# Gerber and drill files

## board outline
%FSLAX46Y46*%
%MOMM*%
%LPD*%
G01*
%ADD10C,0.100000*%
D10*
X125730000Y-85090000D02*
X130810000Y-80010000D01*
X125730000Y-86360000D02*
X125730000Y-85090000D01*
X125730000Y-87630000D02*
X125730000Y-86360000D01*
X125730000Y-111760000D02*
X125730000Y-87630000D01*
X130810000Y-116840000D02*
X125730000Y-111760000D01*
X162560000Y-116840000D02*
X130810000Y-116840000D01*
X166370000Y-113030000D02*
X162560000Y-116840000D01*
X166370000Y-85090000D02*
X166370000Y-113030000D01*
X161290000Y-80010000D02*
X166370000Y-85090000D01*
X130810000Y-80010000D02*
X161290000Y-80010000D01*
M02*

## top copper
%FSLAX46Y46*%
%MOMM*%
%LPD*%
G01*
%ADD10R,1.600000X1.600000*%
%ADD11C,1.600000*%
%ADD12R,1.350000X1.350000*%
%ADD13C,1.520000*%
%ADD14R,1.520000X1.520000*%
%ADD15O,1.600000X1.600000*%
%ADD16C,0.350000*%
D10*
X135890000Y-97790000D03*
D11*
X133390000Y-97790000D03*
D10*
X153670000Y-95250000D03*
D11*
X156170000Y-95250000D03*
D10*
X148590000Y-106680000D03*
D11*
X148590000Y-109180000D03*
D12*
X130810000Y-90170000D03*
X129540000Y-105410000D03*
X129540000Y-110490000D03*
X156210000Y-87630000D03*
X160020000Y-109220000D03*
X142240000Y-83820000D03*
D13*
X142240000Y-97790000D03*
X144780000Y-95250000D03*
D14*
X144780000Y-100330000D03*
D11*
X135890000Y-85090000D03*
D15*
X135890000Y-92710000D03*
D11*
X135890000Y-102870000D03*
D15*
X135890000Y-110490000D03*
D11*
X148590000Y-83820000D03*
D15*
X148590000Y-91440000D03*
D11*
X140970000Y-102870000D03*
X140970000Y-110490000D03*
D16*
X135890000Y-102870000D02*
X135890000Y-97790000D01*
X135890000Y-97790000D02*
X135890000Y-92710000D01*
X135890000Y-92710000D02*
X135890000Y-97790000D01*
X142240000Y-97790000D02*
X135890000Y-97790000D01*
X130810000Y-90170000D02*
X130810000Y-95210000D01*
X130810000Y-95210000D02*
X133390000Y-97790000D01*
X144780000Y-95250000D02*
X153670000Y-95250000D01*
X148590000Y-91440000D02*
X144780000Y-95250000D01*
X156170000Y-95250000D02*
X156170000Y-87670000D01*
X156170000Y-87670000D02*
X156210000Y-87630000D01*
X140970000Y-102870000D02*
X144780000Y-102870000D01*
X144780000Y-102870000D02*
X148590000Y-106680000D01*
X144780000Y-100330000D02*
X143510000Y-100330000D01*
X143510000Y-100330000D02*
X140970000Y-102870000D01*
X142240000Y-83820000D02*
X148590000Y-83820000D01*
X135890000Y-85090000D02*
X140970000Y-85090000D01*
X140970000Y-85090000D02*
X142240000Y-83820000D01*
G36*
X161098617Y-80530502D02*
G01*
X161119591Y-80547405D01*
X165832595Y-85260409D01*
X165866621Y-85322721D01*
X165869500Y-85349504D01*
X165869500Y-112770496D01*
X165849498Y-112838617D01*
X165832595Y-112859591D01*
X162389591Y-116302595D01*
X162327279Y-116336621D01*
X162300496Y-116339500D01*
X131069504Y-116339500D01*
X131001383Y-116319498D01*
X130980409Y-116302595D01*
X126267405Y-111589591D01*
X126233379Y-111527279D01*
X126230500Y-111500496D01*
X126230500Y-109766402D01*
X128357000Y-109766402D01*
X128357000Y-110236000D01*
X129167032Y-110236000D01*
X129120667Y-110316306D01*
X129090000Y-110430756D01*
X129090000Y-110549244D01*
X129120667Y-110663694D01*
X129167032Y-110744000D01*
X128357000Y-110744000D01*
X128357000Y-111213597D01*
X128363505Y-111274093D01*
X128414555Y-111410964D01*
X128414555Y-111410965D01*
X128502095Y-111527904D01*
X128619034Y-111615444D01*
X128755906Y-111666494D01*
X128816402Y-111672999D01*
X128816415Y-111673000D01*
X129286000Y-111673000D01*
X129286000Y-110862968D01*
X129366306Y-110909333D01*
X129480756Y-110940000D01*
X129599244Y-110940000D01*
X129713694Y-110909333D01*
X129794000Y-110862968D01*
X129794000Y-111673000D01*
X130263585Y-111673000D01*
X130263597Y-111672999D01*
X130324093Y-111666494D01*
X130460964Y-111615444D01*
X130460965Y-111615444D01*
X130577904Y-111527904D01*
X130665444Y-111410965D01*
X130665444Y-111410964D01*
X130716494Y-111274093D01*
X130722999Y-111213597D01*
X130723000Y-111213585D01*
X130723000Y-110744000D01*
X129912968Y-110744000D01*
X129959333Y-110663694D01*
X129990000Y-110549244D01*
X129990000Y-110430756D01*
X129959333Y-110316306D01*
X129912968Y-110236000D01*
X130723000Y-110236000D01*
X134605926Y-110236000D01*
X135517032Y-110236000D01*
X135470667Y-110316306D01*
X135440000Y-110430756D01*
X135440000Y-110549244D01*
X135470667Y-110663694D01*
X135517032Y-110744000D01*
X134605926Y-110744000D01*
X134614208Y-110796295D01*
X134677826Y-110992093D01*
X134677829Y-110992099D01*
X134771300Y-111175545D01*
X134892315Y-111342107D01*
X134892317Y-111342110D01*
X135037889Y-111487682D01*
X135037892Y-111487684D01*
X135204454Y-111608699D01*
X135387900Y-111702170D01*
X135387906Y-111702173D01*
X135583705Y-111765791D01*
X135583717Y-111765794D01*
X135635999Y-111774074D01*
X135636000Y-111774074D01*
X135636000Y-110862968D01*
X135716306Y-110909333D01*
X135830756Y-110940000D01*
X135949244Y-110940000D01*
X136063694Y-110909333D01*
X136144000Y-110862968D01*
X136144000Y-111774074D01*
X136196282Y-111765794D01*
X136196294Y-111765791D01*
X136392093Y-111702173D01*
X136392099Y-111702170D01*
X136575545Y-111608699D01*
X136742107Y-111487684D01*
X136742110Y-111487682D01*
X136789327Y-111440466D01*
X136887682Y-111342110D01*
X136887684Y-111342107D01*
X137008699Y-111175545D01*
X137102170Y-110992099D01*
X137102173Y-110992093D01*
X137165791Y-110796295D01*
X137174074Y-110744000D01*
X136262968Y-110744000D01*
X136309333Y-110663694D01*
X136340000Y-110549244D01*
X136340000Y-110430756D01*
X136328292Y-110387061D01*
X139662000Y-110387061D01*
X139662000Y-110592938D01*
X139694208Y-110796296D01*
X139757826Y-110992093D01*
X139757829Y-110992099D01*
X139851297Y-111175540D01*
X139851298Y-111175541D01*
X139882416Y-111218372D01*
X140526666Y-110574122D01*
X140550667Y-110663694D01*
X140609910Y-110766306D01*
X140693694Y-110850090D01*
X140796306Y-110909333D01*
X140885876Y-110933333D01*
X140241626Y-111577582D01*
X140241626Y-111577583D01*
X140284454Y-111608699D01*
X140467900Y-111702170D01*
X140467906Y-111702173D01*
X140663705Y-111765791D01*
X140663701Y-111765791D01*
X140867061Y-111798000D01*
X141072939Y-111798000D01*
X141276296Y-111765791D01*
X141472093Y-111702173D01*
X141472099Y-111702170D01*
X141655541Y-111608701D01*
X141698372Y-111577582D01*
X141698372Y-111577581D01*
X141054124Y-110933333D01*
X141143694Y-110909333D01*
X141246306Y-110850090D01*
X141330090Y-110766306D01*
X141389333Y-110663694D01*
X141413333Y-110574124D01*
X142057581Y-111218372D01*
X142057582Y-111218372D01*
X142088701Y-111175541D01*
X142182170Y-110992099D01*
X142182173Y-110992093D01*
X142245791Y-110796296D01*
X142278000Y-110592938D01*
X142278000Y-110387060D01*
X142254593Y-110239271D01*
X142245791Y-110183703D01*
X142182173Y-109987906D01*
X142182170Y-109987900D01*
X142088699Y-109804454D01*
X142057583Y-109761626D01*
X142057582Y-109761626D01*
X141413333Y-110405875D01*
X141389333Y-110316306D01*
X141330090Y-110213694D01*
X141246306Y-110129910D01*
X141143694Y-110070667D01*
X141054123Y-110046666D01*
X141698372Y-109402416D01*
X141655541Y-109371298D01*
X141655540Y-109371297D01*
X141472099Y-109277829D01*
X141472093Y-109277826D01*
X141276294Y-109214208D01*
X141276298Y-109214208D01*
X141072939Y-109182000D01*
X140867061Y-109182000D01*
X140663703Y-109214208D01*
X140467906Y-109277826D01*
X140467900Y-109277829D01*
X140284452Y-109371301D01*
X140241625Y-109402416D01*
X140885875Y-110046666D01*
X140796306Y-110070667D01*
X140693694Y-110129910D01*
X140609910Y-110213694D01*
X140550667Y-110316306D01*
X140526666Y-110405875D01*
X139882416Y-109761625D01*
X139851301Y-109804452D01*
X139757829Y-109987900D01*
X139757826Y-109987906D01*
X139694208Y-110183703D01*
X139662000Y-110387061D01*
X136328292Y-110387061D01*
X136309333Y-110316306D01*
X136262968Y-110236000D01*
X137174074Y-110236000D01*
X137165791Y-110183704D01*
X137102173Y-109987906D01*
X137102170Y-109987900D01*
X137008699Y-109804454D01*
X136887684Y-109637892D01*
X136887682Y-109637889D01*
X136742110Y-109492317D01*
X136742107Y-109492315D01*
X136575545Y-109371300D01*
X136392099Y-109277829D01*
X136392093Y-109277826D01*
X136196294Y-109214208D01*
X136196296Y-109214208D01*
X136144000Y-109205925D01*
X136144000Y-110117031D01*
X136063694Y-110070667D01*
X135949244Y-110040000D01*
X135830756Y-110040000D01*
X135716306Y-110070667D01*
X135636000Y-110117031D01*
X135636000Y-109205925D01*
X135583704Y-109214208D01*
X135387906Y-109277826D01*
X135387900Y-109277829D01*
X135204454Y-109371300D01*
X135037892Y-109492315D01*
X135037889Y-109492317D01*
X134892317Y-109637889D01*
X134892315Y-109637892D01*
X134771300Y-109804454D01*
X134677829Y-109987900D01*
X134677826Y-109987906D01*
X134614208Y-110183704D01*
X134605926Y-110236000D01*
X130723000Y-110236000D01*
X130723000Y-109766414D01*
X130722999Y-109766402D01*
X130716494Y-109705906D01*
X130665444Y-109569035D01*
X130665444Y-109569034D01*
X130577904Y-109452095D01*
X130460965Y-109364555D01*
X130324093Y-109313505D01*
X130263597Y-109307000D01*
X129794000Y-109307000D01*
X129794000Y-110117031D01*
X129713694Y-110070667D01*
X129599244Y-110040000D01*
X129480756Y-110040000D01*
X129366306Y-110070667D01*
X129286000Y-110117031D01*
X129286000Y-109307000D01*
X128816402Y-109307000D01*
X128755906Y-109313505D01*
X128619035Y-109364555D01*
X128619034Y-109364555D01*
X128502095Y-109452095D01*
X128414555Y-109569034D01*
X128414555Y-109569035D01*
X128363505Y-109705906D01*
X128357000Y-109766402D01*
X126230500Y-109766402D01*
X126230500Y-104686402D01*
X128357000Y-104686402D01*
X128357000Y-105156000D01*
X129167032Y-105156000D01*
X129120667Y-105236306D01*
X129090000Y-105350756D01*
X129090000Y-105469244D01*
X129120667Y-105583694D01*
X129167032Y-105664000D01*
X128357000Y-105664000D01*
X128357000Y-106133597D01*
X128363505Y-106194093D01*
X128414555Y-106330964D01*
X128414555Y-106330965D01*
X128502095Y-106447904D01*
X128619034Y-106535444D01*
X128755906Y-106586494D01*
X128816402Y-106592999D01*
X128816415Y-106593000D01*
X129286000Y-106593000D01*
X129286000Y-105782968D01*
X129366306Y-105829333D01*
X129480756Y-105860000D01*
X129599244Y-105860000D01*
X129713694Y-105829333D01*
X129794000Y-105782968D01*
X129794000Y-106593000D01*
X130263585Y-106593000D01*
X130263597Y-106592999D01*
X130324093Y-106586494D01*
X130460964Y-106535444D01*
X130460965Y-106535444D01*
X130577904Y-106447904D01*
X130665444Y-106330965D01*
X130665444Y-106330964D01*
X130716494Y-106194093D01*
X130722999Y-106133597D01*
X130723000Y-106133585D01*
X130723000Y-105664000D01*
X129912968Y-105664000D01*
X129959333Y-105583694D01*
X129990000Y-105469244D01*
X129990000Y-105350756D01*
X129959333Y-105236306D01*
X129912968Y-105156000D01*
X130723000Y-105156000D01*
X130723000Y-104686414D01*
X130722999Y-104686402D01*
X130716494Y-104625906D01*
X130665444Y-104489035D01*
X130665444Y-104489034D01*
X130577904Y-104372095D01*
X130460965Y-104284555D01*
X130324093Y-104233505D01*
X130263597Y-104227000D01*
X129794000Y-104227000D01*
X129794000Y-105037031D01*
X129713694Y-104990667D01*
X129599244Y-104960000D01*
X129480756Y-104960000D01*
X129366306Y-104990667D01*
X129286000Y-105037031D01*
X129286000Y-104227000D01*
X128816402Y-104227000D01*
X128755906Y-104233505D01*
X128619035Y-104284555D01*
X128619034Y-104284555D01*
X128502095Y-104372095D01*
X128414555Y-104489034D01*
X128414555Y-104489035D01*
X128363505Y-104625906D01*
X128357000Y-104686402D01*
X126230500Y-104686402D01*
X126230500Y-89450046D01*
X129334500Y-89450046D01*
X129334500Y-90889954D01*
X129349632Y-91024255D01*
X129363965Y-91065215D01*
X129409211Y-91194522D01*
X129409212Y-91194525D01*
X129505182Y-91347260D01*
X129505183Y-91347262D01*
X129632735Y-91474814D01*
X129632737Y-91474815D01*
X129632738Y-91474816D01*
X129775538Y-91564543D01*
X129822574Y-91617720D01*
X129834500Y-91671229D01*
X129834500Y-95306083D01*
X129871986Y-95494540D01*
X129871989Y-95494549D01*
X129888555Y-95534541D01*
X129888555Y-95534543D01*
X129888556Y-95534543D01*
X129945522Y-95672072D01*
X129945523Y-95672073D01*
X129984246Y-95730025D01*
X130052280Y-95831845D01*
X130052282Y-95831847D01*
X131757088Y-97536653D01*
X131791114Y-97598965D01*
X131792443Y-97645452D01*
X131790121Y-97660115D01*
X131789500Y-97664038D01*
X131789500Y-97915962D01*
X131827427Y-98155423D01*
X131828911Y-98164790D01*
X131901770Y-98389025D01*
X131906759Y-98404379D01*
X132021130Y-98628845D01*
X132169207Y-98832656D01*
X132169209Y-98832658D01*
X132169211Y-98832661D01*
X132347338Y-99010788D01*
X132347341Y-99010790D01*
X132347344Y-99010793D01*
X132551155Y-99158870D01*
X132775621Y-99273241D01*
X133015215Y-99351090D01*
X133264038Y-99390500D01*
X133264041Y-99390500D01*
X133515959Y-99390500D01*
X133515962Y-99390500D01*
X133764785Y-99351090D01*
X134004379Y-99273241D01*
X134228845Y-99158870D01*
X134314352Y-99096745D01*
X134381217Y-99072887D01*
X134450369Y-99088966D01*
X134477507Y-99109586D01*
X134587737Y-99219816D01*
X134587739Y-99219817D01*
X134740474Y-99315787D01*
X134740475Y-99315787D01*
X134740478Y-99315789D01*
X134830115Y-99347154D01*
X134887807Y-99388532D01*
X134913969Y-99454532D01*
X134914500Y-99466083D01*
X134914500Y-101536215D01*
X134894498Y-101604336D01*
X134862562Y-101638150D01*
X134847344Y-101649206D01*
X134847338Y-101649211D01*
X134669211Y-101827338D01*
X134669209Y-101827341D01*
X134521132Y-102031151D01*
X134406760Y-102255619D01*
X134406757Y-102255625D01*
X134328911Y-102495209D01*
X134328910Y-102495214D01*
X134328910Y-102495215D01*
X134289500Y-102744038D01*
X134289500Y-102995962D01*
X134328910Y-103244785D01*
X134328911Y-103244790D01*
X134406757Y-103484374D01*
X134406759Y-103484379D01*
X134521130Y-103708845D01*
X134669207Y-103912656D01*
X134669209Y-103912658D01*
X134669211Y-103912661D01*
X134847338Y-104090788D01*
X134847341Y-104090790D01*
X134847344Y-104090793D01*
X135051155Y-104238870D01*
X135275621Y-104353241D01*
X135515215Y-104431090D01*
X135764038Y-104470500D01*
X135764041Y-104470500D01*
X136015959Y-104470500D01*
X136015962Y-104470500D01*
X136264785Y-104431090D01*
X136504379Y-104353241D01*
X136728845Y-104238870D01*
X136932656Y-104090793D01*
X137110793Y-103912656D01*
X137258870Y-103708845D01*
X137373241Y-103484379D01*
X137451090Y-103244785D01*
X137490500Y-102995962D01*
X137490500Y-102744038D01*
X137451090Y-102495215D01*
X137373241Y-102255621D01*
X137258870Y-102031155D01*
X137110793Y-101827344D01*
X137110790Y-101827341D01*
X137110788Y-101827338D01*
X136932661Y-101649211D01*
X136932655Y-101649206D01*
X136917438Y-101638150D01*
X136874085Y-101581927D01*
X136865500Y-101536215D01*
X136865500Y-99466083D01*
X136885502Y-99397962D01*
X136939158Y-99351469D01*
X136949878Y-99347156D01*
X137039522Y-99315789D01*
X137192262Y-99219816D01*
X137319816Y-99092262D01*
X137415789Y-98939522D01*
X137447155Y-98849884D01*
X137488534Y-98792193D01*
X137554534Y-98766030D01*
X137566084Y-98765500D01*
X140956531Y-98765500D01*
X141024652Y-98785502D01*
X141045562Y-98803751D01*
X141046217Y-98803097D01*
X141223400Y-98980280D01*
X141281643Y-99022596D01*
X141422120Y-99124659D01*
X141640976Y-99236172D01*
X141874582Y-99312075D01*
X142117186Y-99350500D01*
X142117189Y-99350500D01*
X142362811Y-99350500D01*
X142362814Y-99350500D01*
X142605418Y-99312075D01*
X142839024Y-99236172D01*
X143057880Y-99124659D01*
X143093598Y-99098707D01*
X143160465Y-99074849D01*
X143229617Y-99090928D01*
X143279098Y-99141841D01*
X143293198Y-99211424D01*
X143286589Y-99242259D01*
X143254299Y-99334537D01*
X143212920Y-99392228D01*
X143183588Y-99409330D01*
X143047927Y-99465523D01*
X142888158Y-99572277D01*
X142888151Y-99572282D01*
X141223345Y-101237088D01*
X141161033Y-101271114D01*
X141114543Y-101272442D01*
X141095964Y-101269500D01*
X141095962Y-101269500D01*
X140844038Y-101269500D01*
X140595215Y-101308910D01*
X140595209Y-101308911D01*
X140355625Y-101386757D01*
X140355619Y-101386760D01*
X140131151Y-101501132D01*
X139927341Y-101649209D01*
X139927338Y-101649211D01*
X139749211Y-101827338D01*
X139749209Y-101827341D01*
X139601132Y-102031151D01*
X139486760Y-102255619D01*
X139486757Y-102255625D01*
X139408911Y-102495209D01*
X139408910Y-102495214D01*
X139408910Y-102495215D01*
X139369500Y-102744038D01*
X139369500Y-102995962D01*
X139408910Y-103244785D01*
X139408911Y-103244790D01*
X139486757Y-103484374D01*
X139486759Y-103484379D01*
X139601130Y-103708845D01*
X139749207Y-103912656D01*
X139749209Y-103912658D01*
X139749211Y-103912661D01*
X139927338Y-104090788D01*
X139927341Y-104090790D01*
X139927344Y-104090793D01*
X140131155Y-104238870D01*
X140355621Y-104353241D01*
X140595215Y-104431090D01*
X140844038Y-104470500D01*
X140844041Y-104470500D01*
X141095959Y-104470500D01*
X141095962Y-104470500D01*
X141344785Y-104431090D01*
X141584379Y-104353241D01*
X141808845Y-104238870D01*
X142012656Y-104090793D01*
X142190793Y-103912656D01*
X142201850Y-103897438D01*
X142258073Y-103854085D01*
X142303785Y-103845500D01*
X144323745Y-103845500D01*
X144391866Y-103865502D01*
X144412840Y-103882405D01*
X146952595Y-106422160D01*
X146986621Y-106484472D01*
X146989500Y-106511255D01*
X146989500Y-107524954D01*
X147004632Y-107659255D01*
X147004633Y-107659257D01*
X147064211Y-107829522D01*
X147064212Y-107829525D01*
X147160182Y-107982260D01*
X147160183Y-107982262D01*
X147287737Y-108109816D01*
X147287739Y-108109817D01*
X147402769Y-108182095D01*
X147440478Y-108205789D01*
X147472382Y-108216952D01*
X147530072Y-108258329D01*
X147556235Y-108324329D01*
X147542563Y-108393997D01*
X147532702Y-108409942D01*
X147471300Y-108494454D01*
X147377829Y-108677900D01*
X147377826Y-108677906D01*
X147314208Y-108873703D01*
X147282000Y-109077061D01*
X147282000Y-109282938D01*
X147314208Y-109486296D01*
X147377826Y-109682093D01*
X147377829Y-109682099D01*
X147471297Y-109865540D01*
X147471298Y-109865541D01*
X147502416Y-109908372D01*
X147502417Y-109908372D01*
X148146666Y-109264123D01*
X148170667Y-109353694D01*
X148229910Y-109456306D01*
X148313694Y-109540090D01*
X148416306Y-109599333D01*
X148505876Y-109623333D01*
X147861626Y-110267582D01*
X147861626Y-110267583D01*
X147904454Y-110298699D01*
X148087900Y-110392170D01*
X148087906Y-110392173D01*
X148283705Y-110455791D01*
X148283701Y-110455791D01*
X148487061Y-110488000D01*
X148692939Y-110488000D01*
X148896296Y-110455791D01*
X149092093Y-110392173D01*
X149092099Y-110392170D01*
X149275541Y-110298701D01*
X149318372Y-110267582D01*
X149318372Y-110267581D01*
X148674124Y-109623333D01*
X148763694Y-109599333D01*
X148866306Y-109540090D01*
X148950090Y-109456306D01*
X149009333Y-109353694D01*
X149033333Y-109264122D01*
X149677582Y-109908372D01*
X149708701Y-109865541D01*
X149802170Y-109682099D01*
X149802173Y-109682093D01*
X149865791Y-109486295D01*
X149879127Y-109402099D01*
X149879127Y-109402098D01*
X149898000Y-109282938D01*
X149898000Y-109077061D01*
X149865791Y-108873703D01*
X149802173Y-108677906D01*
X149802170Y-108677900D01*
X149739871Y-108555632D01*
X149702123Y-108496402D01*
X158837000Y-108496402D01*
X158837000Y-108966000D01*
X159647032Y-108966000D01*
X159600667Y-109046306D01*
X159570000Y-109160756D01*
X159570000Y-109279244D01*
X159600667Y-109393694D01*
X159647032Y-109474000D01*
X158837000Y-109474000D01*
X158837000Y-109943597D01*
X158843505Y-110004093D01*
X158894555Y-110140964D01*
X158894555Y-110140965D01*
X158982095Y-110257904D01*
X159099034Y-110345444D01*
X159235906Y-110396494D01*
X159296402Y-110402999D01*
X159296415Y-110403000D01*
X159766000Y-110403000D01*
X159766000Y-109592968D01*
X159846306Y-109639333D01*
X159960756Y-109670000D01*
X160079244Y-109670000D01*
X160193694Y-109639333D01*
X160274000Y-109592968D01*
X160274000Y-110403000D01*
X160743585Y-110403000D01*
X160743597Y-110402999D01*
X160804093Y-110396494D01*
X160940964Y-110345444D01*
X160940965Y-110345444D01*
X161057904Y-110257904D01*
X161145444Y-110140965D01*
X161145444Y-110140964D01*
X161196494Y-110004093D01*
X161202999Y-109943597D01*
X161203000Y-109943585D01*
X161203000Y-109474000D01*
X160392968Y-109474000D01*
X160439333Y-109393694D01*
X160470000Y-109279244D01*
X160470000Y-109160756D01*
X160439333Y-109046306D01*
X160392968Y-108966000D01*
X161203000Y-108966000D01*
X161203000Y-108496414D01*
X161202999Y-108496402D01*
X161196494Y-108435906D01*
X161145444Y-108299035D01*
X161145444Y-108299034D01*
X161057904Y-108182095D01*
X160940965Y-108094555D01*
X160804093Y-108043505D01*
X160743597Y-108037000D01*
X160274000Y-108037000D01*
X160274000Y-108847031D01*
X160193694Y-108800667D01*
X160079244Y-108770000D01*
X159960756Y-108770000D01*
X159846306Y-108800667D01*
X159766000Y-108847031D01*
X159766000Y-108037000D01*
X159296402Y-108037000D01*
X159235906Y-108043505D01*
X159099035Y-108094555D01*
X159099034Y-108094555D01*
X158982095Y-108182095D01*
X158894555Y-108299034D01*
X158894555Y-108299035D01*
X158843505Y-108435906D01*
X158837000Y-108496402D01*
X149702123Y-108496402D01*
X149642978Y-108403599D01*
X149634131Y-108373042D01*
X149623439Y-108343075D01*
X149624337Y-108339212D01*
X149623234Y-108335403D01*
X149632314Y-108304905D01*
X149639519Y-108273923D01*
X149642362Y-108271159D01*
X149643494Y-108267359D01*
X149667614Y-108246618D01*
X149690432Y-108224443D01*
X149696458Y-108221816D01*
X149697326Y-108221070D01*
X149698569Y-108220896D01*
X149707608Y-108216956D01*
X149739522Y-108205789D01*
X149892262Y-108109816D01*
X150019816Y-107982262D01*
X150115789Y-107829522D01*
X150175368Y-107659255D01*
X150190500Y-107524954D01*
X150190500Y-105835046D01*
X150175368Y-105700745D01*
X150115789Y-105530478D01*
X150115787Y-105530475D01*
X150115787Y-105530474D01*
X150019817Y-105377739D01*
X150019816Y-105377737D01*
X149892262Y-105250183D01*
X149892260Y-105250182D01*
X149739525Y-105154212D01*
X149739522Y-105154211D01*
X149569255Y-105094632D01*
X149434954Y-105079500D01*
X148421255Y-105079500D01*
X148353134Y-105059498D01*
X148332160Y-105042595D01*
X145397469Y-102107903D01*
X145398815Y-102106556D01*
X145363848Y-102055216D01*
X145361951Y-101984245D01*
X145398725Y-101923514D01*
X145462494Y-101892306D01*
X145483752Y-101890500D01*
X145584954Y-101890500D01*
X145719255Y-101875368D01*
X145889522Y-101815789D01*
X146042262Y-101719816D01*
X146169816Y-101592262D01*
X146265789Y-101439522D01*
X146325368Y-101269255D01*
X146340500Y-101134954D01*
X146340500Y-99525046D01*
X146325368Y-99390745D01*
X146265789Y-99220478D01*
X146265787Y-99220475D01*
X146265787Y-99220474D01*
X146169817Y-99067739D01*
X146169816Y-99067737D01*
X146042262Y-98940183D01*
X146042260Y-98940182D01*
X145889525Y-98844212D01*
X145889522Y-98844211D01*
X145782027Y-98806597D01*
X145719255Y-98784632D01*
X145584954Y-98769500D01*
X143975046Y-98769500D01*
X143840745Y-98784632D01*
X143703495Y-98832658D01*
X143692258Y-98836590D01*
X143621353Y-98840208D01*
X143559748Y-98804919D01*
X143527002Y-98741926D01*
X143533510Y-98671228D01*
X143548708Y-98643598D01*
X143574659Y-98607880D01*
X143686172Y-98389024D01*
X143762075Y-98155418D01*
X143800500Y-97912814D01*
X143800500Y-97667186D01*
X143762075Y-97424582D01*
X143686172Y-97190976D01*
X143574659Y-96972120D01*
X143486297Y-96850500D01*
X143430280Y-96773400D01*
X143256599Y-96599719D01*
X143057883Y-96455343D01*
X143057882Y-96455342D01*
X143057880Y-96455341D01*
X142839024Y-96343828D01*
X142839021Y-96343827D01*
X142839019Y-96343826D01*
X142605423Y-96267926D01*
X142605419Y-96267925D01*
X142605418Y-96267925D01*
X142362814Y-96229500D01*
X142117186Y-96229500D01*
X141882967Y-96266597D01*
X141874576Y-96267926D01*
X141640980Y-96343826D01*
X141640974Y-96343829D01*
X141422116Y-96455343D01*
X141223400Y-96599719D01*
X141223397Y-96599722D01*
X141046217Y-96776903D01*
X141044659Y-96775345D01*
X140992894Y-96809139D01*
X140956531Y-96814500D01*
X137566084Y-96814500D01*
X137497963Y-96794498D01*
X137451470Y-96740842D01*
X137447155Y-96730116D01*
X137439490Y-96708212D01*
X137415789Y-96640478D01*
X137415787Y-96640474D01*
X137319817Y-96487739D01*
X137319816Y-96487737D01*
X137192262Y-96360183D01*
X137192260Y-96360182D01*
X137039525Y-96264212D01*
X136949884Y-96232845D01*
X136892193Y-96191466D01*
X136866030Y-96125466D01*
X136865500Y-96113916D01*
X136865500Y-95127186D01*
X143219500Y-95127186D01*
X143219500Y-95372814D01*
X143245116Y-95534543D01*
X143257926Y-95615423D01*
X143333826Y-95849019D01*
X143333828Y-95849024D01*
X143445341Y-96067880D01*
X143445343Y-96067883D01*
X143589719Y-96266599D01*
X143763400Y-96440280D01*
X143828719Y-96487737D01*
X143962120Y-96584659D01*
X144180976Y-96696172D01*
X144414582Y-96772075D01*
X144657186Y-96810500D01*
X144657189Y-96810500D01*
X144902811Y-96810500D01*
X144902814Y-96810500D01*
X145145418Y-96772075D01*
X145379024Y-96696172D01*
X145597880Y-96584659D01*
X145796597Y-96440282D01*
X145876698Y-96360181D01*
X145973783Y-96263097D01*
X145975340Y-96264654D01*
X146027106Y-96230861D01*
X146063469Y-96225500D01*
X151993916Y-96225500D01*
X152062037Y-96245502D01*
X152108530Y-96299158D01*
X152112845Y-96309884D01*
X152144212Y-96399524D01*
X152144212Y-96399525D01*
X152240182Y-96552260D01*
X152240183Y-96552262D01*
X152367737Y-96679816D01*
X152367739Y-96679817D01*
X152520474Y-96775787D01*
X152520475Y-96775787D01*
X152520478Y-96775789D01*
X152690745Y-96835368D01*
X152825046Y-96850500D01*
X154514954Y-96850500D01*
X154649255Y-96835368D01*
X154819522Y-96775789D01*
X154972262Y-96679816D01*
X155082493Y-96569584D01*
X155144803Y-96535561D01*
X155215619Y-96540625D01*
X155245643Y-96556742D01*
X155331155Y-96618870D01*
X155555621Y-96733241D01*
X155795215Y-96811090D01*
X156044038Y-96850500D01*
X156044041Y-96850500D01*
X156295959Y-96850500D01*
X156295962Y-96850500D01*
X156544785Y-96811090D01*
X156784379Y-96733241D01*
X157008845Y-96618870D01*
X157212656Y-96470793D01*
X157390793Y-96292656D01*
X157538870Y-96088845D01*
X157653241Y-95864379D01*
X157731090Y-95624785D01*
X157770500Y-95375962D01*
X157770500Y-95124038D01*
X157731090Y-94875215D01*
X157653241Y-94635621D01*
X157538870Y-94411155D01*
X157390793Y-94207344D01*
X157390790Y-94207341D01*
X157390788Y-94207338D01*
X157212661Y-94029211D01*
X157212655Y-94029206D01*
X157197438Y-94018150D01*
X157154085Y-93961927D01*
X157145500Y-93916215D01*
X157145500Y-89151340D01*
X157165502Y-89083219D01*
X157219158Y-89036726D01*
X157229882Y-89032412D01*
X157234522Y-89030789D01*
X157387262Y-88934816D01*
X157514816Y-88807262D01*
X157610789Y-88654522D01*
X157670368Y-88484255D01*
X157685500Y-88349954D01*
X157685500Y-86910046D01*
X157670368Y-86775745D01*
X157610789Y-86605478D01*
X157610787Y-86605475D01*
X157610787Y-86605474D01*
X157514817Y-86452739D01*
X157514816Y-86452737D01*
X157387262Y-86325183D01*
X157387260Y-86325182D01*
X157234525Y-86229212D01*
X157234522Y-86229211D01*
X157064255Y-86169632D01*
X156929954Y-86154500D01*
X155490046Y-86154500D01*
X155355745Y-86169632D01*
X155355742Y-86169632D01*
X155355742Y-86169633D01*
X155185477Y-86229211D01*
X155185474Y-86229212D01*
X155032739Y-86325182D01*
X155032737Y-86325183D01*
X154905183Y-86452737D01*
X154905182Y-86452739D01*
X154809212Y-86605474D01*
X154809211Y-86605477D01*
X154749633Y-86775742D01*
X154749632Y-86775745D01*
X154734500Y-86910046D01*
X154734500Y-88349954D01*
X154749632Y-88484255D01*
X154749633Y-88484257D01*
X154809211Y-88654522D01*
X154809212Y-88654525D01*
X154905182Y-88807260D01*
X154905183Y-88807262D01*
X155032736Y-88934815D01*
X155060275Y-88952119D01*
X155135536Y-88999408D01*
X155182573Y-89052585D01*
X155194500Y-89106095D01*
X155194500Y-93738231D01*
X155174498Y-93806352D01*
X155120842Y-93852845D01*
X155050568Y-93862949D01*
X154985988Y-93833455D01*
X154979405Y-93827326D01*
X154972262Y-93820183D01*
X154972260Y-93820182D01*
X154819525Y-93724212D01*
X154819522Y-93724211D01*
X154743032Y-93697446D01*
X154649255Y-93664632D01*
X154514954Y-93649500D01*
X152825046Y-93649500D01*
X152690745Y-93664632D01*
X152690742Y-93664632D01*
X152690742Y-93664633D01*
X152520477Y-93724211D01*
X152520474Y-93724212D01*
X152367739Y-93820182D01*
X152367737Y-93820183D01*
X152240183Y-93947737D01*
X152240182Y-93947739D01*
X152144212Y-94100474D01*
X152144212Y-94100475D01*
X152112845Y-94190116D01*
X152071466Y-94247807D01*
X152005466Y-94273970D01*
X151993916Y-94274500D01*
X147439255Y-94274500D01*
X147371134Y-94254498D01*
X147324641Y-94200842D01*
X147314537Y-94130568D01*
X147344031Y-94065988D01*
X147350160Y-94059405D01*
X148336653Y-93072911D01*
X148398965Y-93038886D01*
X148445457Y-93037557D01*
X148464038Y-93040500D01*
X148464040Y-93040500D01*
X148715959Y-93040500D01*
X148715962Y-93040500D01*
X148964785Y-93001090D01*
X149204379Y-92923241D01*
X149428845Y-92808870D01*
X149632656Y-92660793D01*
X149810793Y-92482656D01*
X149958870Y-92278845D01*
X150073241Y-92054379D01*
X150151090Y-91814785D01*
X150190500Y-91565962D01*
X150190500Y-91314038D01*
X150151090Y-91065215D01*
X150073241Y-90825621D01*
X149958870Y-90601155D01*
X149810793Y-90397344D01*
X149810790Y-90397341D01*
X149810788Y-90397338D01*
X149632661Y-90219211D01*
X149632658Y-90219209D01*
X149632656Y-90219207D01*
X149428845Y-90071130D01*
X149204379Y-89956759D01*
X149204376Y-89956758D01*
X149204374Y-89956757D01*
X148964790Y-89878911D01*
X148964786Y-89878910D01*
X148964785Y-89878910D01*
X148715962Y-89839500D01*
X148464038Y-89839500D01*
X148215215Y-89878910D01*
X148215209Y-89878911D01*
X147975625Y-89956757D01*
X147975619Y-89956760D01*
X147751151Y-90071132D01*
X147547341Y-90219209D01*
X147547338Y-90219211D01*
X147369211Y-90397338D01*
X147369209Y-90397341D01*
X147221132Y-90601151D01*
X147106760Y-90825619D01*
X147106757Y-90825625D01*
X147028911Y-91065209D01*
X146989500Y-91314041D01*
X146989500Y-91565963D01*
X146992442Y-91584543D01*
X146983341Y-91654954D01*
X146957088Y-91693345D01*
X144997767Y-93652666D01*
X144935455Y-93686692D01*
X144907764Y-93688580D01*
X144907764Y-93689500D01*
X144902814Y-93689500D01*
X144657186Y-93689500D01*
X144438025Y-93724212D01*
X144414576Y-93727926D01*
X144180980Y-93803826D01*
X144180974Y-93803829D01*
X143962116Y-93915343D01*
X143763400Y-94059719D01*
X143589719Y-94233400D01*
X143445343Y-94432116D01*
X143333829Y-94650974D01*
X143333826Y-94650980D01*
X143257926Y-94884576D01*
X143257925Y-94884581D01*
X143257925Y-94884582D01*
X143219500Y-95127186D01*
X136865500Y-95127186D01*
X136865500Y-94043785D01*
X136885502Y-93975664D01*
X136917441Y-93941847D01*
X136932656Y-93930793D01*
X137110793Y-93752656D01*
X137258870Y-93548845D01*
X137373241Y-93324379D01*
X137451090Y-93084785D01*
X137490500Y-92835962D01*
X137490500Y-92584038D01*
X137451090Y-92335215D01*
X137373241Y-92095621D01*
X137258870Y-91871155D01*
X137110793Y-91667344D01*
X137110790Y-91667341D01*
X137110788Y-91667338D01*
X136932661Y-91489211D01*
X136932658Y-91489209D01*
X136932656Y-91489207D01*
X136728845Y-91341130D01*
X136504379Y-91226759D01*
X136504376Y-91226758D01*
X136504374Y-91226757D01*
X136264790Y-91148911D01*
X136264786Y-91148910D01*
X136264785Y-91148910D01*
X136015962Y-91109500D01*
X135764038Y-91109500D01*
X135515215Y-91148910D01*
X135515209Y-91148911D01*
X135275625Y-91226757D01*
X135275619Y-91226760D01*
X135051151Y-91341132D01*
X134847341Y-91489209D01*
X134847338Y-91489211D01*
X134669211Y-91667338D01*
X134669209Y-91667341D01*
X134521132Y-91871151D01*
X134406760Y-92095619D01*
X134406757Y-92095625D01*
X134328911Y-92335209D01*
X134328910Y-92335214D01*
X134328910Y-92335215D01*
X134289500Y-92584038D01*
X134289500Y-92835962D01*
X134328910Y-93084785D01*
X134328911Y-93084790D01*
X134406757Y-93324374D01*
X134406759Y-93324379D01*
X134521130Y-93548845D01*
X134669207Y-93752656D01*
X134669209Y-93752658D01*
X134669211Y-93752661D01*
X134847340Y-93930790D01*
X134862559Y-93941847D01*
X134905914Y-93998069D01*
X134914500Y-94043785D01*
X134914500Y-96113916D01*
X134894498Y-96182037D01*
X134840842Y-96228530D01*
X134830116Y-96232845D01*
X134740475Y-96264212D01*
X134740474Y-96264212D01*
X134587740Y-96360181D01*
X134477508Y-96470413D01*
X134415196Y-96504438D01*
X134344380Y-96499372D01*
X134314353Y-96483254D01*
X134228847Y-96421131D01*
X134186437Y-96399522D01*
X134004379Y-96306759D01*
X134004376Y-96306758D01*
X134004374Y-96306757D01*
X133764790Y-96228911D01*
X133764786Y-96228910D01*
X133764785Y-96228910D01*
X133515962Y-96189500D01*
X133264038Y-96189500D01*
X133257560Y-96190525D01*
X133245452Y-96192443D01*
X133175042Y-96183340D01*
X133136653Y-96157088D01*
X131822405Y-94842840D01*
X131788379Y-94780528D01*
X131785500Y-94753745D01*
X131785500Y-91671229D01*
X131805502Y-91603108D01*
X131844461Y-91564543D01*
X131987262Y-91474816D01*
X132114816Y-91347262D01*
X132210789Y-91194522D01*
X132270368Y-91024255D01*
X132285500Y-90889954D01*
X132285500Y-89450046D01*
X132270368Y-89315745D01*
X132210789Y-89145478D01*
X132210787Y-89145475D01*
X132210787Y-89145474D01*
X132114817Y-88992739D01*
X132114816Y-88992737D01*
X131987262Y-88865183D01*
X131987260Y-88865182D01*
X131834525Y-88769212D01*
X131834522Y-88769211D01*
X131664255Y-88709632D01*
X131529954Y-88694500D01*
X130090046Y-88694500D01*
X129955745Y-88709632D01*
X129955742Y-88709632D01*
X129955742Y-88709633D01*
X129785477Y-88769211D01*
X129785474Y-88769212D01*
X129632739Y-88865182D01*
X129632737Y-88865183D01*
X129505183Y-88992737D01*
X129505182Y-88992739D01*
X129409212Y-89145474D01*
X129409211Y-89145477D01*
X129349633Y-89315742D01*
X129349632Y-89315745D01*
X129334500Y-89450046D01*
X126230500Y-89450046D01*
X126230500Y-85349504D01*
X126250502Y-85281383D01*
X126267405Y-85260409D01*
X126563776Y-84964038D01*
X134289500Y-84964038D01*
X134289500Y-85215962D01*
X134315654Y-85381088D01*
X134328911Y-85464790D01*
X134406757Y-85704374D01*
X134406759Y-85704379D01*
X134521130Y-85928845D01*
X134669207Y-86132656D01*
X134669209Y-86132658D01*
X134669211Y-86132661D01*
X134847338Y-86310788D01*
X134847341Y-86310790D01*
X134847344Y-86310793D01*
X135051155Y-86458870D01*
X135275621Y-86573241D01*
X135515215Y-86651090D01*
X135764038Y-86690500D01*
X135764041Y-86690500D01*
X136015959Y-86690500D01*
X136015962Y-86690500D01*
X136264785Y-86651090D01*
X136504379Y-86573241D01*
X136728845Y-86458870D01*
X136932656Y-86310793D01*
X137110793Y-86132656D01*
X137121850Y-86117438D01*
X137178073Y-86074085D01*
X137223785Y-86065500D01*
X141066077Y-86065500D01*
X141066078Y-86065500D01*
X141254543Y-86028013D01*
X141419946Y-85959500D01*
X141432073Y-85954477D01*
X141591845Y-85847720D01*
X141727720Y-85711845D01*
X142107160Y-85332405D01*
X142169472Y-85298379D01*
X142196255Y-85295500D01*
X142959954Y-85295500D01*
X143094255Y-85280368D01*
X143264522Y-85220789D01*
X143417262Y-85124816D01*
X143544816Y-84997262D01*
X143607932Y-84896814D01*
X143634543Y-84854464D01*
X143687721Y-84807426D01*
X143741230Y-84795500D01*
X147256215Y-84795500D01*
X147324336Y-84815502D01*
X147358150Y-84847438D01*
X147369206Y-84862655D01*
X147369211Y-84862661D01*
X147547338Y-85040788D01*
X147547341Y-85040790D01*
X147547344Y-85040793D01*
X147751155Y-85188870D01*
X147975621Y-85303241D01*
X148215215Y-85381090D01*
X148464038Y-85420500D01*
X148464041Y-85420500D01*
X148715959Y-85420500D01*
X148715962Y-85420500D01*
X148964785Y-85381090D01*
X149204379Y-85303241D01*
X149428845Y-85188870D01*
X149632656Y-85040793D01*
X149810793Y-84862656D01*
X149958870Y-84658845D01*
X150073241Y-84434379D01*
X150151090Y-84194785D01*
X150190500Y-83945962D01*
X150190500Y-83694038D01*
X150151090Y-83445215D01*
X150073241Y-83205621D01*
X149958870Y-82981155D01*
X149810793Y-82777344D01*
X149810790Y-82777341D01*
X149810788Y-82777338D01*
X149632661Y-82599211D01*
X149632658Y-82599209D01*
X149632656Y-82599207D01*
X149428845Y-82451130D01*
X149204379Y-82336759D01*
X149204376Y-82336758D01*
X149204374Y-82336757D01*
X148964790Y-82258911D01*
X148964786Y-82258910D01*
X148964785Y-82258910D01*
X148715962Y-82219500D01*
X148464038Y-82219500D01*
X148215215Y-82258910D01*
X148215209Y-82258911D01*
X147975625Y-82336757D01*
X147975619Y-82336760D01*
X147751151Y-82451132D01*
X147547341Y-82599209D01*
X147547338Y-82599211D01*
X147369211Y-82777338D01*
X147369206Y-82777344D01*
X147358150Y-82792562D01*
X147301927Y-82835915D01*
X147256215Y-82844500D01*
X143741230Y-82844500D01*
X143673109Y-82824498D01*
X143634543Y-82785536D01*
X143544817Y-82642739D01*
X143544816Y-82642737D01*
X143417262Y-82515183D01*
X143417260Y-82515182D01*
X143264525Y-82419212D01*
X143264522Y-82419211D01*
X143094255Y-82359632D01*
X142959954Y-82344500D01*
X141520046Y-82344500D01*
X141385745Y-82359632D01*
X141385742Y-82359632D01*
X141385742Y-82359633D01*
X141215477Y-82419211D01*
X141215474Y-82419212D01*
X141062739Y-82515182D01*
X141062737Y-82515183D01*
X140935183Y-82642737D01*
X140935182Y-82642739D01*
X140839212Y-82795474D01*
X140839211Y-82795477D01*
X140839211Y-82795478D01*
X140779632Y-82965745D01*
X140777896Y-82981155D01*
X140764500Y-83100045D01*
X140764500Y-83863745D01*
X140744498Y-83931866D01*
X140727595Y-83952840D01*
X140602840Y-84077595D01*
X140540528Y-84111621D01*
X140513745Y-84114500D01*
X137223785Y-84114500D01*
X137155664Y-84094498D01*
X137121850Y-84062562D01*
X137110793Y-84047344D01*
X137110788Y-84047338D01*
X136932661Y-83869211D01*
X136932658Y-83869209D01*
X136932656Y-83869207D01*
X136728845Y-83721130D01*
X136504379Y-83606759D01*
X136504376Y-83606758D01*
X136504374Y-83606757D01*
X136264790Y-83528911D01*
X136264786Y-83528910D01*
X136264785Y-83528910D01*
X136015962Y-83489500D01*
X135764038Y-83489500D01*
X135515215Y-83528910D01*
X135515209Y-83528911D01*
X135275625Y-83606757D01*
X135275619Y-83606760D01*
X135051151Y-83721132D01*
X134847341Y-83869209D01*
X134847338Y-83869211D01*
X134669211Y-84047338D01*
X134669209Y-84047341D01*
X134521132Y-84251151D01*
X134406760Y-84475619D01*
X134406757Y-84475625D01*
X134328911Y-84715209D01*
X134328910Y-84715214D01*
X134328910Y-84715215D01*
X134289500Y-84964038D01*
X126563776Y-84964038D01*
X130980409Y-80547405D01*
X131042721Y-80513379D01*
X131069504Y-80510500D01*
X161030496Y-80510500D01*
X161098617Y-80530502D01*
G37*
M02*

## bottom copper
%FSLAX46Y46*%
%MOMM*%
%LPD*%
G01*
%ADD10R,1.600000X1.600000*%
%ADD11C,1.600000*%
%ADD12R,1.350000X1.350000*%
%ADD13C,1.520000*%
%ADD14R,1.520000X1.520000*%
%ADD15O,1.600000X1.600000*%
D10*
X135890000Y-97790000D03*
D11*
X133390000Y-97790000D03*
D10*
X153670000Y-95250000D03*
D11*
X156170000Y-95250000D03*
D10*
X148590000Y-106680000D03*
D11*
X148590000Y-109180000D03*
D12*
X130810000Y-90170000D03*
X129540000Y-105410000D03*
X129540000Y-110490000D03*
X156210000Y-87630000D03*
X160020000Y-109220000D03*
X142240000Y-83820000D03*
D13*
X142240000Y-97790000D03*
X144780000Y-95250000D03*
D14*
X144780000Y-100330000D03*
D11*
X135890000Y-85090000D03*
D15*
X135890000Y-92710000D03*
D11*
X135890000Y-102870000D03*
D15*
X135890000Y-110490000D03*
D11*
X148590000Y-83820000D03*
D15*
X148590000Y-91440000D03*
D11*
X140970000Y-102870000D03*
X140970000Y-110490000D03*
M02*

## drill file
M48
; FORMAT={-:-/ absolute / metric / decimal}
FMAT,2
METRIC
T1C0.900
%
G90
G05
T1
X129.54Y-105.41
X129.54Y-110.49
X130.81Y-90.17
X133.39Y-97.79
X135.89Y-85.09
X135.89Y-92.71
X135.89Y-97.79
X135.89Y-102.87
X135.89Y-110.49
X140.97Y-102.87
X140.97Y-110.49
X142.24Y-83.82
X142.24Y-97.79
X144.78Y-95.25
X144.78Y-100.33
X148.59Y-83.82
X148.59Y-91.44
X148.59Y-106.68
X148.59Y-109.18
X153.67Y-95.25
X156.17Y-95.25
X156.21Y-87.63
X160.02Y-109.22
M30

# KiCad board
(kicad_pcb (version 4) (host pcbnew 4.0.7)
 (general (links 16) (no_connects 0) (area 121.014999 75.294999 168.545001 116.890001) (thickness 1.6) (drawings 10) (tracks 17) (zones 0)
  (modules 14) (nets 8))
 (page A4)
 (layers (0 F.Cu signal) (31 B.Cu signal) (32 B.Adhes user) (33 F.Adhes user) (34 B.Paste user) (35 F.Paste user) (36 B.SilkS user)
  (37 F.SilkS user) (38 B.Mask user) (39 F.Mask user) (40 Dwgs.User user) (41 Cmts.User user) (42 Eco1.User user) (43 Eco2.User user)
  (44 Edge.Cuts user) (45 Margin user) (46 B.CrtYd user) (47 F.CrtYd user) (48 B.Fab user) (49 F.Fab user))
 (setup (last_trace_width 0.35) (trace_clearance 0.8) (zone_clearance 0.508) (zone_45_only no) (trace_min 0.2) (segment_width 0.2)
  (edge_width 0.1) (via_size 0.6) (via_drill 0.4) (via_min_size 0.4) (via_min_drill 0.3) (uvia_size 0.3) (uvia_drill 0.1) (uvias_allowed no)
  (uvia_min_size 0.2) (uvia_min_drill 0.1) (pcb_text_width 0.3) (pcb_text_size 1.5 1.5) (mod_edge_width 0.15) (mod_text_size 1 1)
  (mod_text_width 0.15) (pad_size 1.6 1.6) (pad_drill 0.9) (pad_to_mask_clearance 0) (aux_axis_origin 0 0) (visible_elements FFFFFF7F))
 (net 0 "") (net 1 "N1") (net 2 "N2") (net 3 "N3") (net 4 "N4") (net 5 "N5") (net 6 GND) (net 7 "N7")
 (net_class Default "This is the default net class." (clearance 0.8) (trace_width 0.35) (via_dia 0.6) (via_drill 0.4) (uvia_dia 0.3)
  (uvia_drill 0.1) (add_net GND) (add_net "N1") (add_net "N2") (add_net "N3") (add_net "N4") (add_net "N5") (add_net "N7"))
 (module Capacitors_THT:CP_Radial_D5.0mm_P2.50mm (layer F.Cu) (at 135.89 97.79 180)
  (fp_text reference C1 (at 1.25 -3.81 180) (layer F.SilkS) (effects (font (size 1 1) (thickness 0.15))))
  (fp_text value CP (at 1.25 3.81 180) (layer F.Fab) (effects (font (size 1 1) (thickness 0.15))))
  (pad 1 thru_hole rect (at 0 0 180) (size 1.6 1.6) (drill 0.9) (layers *.Cu *.Mask) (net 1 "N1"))
  (pad 2 thru_hole circle (at 2.5 0 180) (size 1.6 1.6) (drill 0.9) (layers *.Cu *.Mask) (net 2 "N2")))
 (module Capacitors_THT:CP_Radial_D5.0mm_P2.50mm (layer F.Cu) (at 153.67 95.25)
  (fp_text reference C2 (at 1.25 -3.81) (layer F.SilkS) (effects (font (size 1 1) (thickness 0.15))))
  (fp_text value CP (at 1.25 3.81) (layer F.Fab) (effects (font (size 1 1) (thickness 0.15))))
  (pad 1 thru_hole rect (at 0 0) (size 1.6 1.6) (drill 0.9) (layers *.Cu *.Mask) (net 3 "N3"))
  (pad 2 thru_hole circle (at 2.5 0) (size 1.6 1.6) (drill 0.9) (layers *.Cu *.Mask) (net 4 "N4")))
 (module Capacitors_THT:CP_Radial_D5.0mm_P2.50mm (layer F.Cu) (at 148.59 106.68 270)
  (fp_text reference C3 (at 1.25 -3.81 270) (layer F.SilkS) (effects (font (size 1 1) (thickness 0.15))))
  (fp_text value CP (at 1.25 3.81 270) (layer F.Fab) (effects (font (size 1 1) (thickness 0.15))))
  (pad 1 thru_hole rect (at 0 0 270) (size 1.6 1.6) (drill 0.9) (layers *.Cu *.Mask) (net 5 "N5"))
  (pad 2 thru_hole circle (at 2.5 0 270) (size 1.6 1.6) (drill 0.9) (layers *.Cu *.Mask) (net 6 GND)))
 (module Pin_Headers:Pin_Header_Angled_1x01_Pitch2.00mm (layer F.Cu) (at 130.81 90.17 180)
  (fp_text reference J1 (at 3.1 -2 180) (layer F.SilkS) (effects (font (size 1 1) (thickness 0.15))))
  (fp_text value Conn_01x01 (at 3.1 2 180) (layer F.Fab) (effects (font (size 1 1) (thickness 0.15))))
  (pad 1 thru_hole rect (at 0 0 180) (size 1.35 1.35) (drill 0.9) (layers *.Cu *.Mask) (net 2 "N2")))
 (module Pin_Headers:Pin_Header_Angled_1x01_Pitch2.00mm (layer F.Cu) (at 129.54 105.41 180)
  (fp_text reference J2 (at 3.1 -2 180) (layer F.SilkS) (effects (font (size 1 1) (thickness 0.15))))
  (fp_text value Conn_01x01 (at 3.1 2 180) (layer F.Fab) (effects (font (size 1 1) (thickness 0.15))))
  (pad 1 thru_hole rect (at 0 0 180) (size 1.35 1.35) (drill 0.9) (layers *.Cu *.Mask) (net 6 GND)))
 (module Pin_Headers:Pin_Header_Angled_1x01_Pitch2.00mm (layer F.Cu) (at 129.54 110.49 180)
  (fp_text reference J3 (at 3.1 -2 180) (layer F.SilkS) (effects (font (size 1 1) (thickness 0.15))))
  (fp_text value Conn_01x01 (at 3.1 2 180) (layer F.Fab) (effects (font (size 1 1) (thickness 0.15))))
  (pad 1 thru_hole rect (at 0 0 180) (size 1.35 1.35) (drill 0.9) (layers *.Cu *.Mask) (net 6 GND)))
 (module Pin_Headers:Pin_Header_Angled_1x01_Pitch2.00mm (layer F.Cu) (at 156.21 87.63)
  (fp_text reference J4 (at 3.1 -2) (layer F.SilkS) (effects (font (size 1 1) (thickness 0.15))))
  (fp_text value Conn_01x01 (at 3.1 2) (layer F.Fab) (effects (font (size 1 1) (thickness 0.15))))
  (pad 1 thru_hole rect (at 0 0) (size 1.35 1.35) (drill 0.9) (layers *.Cu *.Mask) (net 4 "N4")))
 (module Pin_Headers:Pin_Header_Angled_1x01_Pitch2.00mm (layer F.Cu) (at 160.02 109.22)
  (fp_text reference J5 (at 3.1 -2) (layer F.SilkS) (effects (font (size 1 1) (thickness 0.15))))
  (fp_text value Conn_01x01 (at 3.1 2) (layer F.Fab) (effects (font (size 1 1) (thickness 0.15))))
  (pad 1 thru_hole rect (at 0 0) (size 1.35 1.35) (drill 0.9) (layers *.Cu *.Mask) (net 6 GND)))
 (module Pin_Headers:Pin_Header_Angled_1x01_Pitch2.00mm (layer F.Cu) (at 142.24 83.82 90)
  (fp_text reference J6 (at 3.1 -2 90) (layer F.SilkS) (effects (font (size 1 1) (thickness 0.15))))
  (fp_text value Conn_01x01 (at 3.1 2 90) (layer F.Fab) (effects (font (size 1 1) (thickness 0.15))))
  (pad 1 thru_hole rect (at 0 0 90) (size 1.35 1.35) (drill 0.9) (layers *.Cu *.Mask) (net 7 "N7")))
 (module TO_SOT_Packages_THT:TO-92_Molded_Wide (layer F.Cu) (at 144.78 100.33 90)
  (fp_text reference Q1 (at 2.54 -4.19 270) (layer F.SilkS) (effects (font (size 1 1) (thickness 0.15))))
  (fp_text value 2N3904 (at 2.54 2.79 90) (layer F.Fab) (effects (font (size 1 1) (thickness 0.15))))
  (pad 2 thru_hole circle (at 2.54 -2.54 180) (size 1.52 1.52) (drill 0.9) (layers *.Cu *.Mask) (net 1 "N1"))
  (pad 3 thru_hole circle (at 5.08 0 180) (size 1.52 1.52) (drill 0.9) (layers *.Cu *.Mask) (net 3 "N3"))
  (pad 1 thru_hole rect (at 0 0 180) (size 1.52 1.52) (drill 0.9) (layers *.Cu *.Mask) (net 5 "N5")))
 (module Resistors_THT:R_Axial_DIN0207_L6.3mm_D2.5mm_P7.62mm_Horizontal (layer F.Cu) (at 135.89 85.09 270)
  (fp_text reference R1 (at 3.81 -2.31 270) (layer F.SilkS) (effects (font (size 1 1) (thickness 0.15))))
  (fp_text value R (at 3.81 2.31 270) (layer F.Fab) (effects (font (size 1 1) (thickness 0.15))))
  (pad 1 thru_hole circle (at 0 0 270) (size 1.6 1.6) (drill 0.9) (layers *.Cu *.Mask) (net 7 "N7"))
  (pad 2 thru_hole oval (at 7.62 0 270) (size 1.6 1.6) (drill 0.9) (layers *.Cu *.Mask) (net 1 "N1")))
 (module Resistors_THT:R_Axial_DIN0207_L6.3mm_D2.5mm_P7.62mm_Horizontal (layer F.Cu) (at 135.89 102.87 270)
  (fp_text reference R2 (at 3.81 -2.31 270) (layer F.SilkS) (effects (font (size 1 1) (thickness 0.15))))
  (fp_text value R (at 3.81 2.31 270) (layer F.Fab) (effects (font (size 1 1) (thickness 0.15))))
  (pad 1 thru_hole circle (at 0 0 270) (size 1.6 1.6) (drill 0.9) (layers *.Cu *.Mask) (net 1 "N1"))
  (pad 2 thru_hole oval (at 7.62 0 270) (size 1.6 1.6) (drill 0.9) (layers *.Cu *.Mask) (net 6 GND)))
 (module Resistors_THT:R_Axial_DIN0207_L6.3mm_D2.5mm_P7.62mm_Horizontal (layer F.Cu) (at 148.59 83.82 270)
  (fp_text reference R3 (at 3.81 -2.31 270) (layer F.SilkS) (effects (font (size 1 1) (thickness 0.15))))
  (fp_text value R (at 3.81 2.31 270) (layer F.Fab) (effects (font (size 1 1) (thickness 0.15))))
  (pad 1 thru_hole circle (at 0 0 270) (size 1.6 1.6) (drill 0.9) (layers *.Cu *.Mask) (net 7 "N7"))
  (pad 2 thru_hole oval (at 7.62 0 270) (size 1.6 1.6) (drill 0.9) (layers *.Cu *.Mask) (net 3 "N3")))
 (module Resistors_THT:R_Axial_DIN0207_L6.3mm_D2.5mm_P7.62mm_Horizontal (layer F.Cu) (at 140.97 102.87 270)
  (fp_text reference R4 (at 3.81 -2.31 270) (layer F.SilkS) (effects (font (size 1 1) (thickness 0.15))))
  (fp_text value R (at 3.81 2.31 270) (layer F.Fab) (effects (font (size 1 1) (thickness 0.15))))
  (pad 1 thru_hole circle (at 0 0 270) (size 1.6 1.6) (drill 0.9) (layers *.Cu *.Mask) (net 5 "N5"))
  (pad 2 thru_hole circle (at 7.62 0 270) (size 1.6 1.6) (drill 0.9) (layers *.Cu *.Mask) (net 6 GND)))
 (gr_line (start 125.73 85.09) (end 130.81 80.01) (angle 90) (layer Edge.Cuts) (width 0.1))
 (gr_line (start 125.73 86.36) (end 125.73 85.09) (angle 90) (layer Edge.Cuts) (width 0.1))
 (gr_line (start 125.73 87.63) (end 125.73 86.36) (angle 90) (layer Edge.Cuts) (width 0.1))
 (gr_line (start 125.73 111.76) (end 125.73 87.63) (angle 90) (layer Edge.Cuts) (width 0.1))
 (gr_line (start 130.81 116.84) (end 125.73 111.76) (angle 90) (layer Edge.Cuts) (width 0.1))
 (gr_line (start 162.56 116.84) (end 130.81 116.84) (angle 90) (layer Edge.Cuts) (width 0.1))
 (gr_line (start 166.37 113.03) (end 162.56 116.84) (angle 90) (layer Edge.Cuts) (width 0.1))
 (gr_line (start 166.37 85.09) (end 166.37 113.03) (angle 90) (layer Edge.Cuts) (width 0.1))
 (gr_line (start 161.29 80.01) (end 166.37 85.09) (angle 90) (layer Edge.Cuts) (width 0.1))
 (gr_line (start 130.81 80.01) (end 161.29 80.01) (angle 90) (layer Edge.Cuts) (width 0.1))
 (segment (start 135.89 102.87) (end 135.89 97.79) (width 0.35) (layer F.Cu) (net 1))
 (segment (start 135.89 97.79) (end 135.89 92.71) (width 0.35) (layer F.Cu) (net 1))
 (segment (start 135.89 92.71) (end 135.89 97.79) (width 0.35) (layer F.Cu) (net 1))
 (segment (start 142.24 97.79) (end 135.89 97.79) (width 0.35) (layer F.Cu) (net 1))
 (segment (start 130.81 90.17) (end 130.81 95.21) (width 0.35) (layer F.Cu) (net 2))
 (segment (start 130.81 95.21) (end 133.39 97.79) (width 0.35) (layer F.Cu) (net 2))
 (segment (start 144.78 95.25) (end 153.67 95.25) (width 0.35) (layer F.Cu) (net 3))
 (segment (start 148.59 91.44) (end 144.78 95.25) (width 0.35) (layer F.Cu) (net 3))
 (segment (start 156.17 95.25) (end 156.17 87.67) (width 0.35) (layer F.Cu) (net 4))
 (segment (start 156.17 87.67) (end 156.21 87.63) (width 0.35) (layer F.Cu) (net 4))
 (segment (start 140.97 102.87) (end 144.78 102.87) (width 0.35) (layer F.Cu) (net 5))
 (segment (start 144.78 102.87) (end 148.59 106.68) (width 0.35) (layer F.Cu) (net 5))
 (segment (start 144.78 100.33) (end 143.51 100.33) (width 0.35) (layer F.Cu) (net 5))
 (segment (start 143.51 100.33) (end 140.97 102.87) (width 0.35) (layer F.Cu) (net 5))
 (segment (start 142.24 83.82) (end 148.59 83.82) (width 0.35) (layer F.Cu) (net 7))
 (segment (start 135.89 85.09) (end 140.97 85.09) (width 0.35) (layer F.Cu) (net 7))
 (segment (start 140.97 85.09) (end 142.24 83.82) (width 0.35) (layer F.Cu) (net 7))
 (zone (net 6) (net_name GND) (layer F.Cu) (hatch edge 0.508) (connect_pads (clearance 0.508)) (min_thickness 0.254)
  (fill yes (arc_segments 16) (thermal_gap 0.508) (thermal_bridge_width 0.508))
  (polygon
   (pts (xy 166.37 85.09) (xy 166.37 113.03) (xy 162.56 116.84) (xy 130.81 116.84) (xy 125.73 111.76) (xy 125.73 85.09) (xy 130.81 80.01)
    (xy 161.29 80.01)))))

